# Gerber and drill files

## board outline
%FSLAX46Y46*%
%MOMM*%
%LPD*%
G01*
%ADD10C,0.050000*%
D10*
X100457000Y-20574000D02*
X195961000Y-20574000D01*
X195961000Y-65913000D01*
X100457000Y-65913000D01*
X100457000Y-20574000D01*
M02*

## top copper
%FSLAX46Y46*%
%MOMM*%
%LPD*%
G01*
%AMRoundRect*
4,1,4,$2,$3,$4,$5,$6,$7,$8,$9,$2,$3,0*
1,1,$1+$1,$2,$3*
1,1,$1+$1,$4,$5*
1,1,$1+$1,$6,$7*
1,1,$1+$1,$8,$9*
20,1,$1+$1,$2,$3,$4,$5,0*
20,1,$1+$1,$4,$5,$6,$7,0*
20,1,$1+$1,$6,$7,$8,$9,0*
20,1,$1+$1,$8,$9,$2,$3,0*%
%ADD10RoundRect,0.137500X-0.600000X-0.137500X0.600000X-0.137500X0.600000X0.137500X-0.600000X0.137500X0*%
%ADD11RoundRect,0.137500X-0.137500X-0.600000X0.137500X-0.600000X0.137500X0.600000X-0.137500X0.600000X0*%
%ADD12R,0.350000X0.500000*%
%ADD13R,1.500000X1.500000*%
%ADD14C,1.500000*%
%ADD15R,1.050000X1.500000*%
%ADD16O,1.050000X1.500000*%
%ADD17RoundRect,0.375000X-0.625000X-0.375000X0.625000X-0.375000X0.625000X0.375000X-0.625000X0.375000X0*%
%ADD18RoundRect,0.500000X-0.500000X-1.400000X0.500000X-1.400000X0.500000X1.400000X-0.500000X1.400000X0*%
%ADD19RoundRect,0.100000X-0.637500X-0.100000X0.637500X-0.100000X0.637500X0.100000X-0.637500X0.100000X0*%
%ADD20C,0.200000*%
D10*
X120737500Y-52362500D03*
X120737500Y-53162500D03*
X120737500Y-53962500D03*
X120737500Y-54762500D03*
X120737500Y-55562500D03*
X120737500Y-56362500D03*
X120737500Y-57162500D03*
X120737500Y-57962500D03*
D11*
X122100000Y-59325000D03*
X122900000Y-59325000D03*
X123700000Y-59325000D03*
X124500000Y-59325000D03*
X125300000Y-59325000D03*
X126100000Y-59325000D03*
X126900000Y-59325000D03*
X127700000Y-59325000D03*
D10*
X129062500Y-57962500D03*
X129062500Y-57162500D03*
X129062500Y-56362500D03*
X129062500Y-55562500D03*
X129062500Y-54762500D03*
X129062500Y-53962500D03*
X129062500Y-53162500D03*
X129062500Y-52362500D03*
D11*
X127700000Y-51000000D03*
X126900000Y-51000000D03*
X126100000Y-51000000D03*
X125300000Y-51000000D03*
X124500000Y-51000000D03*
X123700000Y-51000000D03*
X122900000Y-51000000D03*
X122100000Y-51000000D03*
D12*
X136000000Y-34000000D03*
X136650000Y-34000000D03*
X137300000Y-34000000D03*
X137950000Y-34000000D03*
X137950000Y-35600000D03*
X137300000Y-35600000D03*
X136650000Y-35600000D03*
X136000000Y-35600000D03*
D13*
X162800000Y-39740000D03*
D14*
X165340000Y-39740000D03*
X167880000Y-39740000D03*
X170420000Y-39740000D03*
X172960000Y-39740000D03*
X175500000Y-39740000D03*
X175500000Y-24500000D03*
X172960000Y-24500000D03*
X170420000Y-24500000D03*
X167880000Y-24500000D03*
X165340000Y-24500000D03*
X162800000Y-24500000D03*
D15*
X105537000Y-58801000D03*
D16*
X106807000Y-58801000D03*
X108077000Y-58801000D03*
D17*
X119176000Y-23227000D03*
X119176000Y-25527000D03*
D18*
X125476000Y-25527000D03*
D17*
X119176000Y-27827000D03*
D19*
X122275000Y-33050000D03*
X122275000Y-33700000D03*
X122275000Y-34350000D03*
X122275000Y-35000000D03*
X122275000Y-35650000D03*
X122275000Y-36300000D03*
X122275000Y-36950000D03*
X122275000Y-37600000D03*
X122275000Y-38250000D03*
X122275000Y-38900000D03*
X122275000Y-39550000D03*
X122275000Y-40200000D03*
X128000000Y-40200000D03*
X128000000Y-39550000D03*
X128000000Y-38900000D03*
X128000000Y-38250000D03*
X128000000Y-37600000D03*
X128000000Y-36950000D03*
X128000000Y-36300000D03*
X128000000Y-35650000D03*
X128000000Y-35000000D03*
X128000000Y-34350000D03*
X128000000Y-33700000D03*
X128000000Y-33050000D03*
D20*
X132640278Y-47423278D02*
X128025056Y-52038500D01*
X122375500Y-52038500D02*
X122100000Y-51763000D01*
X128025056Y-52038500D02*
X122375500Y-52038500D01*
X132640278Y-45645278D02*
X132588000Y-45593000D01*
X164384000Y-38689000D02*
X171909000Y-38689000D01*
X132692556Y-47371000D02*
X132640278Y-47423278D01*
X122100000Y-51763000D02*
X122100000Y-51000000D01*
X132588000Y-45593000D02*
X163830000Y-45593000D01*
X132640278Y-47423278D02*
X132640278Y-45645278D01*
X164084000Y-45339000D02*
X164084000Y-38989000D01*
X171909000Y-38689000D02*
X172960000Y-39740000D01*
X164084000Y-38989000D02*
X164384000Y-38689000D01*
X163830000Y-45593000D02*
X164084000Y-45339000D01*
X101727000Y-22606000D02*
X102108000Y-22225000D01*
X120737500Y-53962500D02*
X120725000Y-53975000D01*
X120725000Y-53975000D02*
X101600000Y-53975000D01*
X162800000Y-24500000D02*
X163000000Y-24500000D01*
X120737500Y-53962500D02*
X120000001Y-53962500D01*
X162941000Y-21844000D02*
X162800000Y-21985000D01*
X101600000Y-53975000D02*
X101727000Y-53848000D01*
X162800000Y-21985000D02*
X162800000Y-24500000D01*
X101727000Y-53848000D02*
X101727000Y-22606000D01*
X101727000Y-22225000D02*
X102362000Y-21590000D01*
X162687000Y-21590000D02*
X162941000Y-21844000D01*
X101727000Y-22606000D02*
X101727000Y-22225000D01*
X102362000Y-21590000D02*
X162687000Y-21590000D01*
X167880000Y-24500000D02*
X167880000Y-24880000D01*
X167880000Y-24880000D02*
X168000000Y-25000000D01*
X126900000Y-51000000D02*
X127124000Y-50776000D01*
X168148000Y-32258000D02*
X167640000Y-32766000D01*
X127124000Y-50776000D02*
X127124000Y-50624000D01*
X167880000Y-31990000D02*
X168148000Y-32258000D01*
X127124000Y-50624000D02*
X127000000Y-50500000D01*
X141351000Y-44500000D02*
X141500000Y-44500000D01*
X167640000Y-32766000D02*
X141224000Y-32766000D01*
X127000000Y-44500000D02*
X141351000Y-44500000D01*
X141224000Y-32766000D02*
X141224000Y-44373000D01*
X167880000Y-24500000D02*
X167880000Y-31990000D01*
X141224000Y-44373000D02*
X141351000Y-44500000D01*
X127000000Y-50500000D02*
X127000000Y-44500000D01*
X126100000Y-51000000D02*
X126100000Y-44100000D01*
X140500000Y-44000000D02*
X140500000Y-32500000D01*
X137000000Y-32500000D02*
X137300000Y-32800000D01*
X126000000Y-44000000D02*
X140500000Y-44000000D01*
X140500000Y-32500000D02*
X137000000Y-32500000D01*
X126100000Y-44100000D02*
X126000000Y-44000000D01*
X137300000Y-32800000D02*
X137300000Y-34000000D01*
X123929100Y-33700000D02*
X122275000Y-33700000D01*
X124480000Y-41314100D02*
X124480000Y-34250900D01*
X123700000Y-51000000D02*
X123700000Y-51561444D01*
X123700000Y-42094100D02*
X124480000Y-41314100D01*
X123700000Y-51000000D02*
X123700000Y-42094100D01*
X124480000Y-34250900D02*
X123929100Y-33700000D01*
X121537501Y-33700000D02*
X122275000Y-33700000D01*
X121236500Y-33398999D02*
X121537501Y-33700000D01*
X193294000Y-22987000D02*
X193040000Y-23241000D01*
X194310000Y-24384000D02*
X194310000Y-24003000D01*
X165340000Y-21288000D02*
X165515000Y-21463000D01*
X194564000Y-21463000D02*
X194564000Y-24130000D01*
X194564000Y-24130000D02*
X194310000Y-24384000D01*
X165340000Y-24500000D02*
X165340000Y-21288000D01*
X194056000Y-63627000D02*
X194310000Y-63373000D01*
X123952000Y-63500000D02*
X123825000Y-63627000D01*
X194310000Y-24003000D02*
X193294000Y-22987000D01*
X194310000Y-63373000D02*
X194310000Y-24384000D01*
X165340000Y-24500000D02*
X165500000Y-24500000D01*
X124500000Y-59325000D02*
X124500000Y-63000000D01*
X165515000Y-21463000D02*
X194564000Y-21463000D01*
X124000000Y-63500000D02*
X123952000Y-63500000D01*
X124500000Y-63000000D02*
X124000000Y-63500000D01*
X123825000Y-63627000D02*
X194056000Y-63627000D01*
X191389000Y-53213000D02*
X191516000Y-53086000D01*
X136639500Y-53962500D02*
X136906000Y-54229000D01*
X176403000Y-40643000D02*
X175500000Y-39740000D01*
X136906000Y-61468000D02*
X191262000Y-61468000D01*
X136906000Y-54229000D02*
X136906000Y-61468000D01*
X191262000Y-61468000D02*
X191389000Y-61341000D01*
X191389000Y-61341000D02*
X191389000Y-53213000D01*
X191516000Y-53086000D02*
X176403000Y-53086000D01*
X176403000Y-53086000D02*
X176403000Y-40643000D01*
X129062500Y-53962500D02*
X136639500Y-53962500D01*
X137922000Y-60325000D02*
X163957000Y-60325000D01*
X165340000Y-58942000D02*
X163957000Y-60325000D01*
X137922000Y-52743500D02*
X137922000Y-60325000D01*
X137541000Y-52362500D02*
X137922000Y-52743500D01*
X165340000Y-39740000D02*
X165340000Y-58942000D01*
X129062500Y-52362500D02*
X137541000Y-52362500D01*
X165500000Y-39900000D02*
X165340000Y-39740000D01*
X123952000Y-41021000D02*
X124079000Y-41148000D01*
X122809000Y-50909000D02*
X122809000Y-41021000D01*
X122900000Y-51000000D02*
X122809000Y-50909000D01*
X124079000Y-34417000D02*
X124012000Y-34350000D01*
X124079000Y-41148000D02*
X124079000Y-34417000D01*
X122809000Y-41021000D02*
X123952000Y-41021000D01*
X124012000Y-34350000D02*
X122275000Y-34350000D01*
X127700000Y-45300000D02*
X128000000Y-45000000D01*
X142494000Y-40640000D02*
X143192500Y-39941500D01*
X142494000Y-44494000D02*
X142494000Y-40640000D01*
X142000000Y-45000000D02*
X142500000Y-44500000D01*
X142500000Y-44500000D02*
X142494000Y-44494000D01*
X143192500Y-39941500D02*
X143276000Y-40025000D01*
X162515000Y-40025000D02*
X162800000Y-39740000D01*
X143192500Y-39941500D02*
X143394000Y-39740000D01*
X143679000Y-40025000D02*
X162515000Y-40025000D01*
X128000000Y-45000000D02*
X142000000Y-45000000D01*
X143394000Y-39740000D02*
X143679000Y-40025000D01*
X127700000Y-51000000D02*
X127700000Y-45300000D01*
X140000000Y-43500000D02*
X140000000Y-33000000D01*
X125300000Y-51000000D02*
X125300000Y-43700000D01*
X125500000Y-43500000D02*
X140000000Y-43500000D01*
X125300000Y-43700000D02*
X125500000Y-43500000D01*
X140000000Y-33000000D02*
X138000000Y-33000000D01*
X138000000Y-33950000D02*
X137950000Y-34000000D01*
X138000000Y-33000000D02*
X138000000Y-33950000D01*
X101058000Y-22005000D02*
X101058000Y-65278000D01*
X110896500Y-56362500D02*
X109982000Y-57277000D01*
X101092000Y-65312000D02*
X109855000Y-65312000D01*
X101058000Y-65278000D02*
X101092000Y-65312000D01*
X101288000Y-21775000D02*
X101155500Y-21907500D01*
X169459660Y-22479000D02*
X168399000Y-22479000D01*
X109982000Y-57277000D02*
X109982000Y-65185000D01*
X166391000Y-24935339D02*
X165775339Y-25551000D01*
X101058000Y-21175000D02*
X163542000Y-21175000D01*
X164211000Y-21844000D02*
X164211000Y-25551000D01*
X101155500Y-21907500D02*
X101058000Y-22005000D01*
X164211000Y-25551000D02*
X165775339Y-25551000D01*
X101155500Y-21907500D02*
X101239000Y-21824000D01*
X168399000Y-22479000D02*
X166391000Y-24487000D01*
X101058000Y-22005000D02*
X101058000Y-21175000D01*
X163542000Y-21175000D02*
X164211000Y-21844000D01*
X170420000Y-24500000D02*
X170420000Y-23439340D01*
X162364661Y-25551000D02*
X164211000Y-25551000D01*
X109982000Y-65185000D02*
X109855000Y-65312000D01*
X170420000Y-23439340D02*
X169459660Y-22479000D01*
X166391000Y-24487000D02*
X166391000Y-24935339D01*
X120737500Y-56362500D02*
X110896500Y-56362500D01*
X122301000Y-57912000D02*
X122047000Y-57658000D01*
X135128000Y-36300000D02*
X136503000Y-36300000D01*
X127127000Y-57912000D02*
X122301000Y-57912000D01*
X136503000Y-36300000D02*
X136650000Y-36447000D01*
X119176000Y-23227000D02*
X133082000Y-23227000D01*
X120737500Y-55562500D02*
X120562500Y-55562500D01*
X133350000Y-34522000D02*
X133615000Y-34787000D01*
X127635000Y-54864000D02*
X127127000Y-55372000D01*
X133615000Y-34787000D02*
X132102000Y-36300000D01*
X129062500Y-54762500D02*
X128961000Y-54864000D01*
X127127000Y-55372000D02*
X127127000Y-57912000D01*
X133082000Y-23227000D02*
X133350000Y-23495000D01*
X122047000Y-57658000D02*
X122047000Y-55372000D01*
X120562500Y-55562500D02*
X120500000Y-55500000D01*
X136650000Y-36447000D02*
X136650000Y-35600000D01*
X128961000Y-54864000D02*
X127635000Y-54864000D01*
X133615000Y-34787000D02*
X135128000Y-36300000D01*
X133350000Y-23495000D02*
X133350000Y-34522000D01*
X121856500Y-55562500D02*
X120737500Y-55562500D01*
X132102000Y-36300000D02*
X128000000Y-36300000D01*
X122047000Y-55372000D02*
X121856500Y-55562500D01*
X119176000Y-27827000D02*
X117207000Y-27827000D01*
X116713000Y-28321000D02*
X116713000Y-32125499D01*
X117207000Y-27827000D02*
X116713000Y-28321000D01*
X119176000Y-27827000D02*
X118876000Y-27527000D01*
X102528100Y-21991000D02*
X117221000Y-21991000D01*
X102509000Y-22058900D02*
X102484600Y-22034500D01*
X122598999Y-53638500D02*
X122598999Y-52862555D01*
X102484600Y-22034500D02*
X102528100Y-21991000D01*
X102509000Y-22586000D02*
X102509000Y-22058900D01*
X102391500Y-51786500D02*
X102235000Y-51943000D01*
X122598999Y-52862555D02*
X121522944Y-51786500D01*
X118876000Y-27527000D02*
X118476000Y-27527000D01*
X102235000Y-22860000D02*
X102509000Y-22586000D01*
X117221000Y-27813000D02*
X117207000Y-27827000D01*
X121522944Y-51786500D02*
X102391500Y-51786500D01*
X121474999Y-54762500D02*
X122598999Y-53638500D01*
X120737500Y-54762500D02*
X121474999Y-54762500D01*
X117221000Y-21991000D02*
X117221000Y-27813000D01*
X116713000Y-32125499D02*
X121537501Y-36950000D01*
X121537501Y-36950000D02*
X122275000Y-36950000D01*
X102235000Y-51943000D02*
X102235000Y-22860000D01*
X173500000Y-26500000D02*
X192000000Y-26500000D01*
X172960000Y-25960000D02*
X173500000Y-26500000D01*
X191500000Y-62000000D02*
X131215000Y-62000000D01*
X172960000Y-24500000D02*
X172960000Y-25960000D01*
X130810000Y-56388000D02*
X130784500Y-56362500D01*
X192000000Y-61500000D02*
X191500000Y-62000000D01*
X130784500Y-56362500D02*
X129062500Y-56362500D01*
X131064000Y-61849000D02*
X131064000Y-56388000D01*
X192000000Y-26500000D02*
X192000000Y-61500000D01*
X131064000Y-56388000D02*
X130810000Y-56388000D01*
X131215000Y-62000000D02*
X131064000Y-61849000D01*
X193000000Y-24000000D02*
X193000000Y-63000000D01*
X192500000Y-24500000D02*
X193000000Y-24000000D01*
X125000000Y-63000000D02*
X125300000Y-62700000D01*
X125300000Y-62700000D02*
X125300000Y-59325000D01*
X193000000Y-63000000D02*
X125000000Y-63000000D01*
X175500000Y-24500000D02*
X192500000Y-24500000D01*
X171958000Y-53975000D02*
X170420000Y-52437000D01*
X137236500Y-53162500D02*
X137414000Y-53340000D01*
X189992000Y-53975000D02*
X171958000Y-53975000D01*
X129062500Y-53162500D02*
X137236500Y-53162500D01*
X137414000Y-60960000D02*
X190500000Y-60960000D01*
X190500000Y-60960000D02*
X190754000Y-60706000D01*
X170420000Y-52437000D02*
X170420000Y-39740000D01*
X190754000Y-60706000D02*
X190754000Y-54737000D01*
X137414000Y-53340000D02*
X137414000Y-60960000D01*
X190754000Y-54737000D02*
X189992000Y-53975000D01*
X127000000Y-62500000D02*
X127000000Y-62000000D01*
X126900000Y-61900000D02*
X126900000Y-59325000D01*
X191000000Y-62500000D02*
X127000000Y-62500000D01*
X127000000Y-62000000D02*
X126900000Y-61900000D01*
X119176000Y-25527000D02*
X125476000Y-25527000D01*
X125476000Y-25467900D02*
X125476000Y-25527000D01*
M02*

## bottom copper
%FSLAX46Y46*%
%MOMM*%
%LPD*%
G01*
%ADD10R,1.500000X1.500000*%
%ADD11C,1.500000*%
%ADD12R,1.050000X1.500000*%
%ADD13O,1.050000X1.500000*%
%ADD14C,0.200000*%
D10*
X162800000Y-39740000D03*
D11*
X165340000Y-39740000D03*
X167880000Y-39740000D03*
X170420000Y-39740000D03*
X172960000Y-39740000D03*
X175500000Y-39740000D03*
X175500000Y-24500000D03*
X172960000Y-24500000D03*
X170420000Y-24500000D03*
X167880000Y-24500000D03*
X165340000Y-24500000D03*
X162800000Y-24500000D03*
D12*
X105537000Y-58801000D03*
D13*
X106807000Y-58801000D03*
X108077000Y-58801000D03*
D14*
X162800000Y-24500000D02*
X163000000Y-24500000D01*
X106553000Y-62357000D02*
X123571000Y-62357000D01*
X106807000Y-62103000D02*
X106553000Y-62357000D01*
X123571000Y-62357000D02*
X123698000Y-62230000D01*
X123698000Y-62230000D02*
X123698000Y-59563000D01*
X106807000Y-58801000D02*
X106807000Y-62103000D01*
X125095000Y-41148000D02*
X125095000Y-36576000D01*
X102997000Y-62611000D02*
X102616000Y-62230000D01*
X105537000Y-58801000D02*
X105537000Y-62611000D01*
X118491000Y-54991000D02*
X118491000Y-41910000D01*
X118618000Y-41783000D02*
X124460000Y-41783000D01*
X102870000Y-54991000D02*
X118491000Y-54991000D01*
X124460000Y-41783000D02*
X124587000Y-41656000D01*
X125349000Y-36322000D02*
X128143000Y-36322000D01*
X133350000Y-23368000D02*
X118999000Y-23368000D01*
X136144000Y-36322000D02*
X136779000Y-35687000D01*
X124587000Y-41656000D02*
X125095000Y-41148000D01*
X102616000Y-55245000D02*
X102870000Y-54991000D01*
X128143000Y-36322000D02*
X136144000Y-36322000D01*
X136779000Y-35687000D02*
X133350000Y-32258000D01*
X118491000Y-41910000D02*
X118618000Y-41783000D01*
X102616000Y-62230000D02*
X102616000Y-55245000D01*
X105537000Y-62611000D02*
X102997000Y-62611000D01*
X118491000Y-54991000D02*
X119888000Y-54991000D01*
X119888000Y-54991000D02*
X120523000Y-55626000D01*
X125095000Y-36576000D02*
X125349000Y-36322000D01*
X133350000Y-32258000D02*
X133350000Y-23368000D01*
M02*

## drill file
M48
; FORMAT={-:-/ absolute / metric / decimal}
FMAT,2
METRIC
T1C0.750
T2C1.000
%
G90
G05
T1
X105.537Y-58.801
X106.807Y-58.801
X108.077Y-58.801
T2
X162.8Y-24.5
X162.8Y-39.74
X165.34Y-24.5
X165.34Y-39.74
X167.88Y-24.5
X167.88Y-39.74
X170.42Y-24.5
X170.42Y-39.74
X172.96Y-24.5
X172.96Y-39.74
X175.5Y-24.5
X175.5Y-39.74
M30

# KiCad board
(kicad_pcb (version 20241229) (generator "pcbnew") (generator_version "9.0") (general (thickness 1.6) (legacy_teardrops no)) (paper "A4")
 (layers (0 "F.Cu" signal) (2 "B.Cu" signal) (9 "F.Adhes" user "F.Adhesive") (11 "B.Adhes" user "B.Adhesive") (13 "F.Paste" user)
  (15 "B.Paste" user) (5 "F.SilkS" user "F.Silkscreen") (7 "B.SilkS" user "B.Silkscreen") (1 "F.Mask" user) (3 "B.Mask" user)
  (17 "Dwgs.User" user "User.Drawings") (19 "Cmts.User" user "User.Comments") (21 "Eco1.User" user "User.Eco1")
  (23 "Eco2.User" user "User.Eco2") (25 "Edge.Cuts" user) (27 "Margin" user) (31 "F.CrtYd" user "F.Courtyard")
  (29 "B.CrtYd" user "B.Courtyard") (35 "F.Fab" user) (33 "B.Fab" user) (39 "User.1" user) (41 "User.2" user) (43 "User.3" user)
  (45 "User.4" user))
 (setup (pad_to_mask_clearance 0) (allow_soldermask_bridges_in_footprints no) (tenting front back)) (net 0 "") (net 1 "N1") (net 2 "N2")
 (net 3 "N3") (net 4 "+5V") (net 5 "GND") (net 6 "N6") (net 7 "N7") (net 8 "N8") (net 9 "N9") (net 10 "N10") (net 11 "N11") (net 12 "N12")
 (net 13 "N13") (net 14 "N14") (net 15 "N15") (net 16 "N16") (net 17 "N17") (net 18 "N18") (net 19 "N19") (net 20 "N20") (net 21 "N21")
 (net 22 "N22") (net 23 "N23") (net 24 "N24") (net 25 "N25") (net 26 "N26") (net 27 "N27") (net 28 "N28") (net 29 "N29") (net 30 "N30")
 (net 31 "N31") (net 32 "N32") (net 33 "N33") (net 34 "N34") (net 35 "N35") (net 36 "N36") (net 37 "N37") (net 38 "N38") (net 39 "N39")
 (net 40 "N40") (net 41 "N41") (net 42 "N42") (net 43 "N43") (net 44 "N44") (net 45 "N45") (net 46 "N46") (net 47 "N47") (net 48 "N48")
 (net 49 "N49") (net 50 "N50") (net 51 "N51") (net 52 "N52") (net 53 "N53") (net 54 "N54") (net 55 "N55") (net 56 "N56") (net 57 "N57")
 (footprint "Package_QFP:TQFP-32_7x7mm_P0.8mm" (layer "F.Cu") (at 124.9 55.1625)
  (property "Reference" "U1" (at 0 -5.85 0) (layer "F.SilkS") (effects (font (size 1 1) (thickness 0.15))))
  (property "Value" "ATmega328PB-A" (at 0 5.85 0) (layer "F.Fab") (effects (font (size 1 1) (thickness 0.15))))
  (pad "1" smd roundrect (at -4.1625 -2.8) (size 1.475 0.55) (layers "F.Cu" "F.Mask" "F.Paste") (roundrect_rratio 0.25) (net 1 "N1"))
  (pad "2" smd roundrect (at -4.1625 -2) (size 1.475 0.55) (layers "F.Cu" "F.Mask" "F.Paste") (roundrect_rratio 0.25) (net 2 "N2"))
  (pad "3" smd roundrect (at -4.1625 -1.2) (size 1.475 0.55) (layers "F.Cu" "F.Mask" "F.Paste") (roundrect_rratio 0.25) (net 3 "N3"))
  (pad "4" smd roundrect (at -4.1625 -0.4) (size 1.475 0.55) (layers "F.Cu" "F.Mask" "F.Paste") (roundrect_rratio 0.25) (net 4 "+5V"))
  (pad "5" smd roundrect (at -4.1625 0.4) (size 1.475 0.55) (layers "F.Cu" "F.Mask" "F.Paste") (roundrect_rratio 0.25) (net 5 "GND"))
  (pad "6" smd roundrect (at -4.1625 1.2) (size 1.475 0.55) (layers "F.Cu" "F.Mask" "F.Paste") (roundrect_rratio 0.25) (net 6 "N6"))
  (pad "7" smd roundrect (at -4.1625 2) (size 1.475 0.55) (layers "F.Cu" "F.Mask" "F.Paste") (roundrect_rratio 0.25) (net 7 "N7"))
  (pad "8" smd roundrect (at -4.1625 2.8) (size 1.475 0.55) (layers "F.Cu" "F.Mask" "F.Paste") (roundrect_rratio 0.25) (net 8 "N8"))
  (pad "9" smd roundrect (at -2.8 4.1625) (size 0.55 1.475) (layers "F.Cu" "F.Mask" "F.Paste") (roundrect_rratio 0.25) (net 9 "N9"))
  (pad "10" smd roundrect (at -2 4.1625) (size 0.55 1.475) (layers "F.Cu" "F.Mask" "F.Paste") (roundrect_rratio 0.25) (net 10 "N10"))
  (pad "11" smd roundrect (at -1.2 4.1625) (size 0.55 1.475) (layers "F.Cu" "F.Mask" "F.Paste") (roundrect_rratio 0.25) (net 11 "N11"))
  (pad "12" smd roundrect (at -0.4 4.1625) (size 0.55 1.475) (layers "F.Cu" "F.Mask" "F.Paste") (roundrect_rratio 0.25) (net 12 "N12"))
  (pad "13" smd roundrect (at 0.4 4.1625) (size 0.55 1.475) (layers "F.Cu" "F.Mask" "F.Paste") (roundrect_rratio 0.25) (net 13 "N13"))
  (pad "14" smd roundrect (at 1.2 4.1625) (size 0.55 1.475) (layers "F.Cu" "F.Mask" "F.Paste") (roundrect_rratio 0.25) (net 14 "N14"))
  (pad "15" smd roundrect (at 2 4.1625) (size 0.55 1.475) (layers "F.Cu" "F.Mask" "F.Paste") (roundrect_rratio 0.25) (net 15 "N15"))
  (pad "16" smd roundrect (at 2.8 4.1625) (size 0.55 1.475) (layers "F.Cu" "F.Mask" "F.Paste") (roundrect_rratio 0.25) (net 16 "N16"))
  (pad "17" smd roundrect (at 4.1625 2.8) (size 1.475 0.55) (layers "F.Cu" "F.Mask" "F.Paste") (roundrect_rratio 0.25) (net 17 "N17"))
  (pad "18" smd roundrect (at 4.1625 2) (size 1.475 0.55) (layers "F.Cu" "F.Mask" "F.Paste") (roundrect_rratio 0.25) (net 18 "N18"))
  (pad "19" smd roundrect (at 4.1625 1.2) (size 1.475 0.55) (layers "F.Cu" "F.Mask" "F.Paste") (roundrect_rratio 0.25) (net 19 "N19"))
  (pad "20" smd roundrect (at 4.1625 0.4) (size 1.475 0.55) (layers "F.Cu" "F.Mask" "F.Paste") (roundrect_rratio 0.25) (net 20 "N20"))
  (pad "21" smd roundrect (at 4.1625 -0.4) (size 1.475 0.55) (layers "F.Cu" "F.Mask" "F.Paste") (roundrect_rratio 0.25) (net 5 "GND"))
  (pad "22" smd roundrect (at 4.1625 -1.2) (size 1.475 0.55) (layers "F.Cu" "F.Mask" "F.Paste") (roundrect_rratio 0.25) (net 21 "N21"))
  (pad "23" smd roundrect (at 4.1625 -2) (size 1.475 0.55) (layers "F.Cu" "F.Mask" "F.Paste") (roundrect_rratio 0.25) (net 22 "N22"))
  (pad "24" smd roundrect (at 4.1625 -2.8) (size 1.475 0.55) (layers "F.Cu" "F.Mask" "F.Paste") (roundrect_rratio 0.25) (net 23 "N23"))
  (pad "25" smd roundrect (at 2.8 -4.1625) (size 0.55 1.475) (layers "F.Cu" "F.Mask" "F.Paste") (roundrect_rratio 0.25) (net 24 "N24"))
  (pad "26" smd roundrect (at 2 -4.1625) (size 0.55 1.475) (layers "F.Cu" "F.Mask" "F.Paste") (roundrect_rratio 0.25) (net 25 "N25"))
  (pad "27" smd roundrect (at 1.2 -4.1625) (size 0.55 1.475) (layers "F.Cu" "F.Mask" "F.Paste") (roundrect_rratio 0.25) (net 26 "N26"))
  (pad "28" smd roundrect (at 0.4 -4.1625) (size 0.55 1.475) (layers "F.Cu" "F.Mask" "F.Paste") (roundrect_rratio 0.25) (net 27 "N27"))
  (pad "29" smd roundrect (at -0.4 -4.1625) (size 0.55 1.475) (layers "F.Cu" "F.Mask" "F.Paste") (roundrect_rratio 0.25) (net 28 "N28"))
  (pad "30" smd roundrect (at -1.2 -4.1625) (size 0.55 1.475) (layers "F.Cu" "F.Mask" "F.Paste") (roundrect_rratio 0.25) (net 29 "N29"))
  (pad "31" smd roundrect (at -2 -4.1625) (size 0.55 1.475) (layers "F.Cu" "F.Mask" "F.Paste") (roundrect_rratio 0.25) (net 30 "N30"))
  (pad "32" smd roundrect (at -2.8 -4.1625) (size 0.55 1.475) (layers "F.Cu" "F.Mask" "F.Paste") (roundrect_rratio 0.25) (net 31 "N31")))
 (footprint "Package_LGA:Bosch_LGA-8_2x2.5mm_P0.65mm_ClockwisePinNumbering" (layer "F.Cu") (at 136.975 34.8)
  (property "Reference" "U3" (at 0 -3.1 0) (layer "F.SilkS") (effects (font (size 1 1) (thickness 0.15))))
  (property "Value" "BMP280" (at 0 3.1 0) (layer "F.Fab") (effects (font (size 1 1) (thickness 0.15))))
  (pad "1" smd rect (at -0.975 -0.8 90) (size 0.5 0.35) (layers "F.Cu" "F.Mask" "F.Paste") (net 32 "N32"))
  (pad "2" smd rect (at -0.325 -0.8 90) (size 0.5 0.35) (layers "F.Cu" "F.Mask" "F.Paste") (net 32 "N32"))
  (pad "3" smd rect (at 0.325 -0.8 90) (size 0.5 0.35) (layers "F.Cu" "F.Mask" "F.Paste") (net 26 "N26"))
  (pad "4" smd rect (at 0.975 -0.8 90) (size 0.5 0.35) (layers "F.Cu" "F.Mask" "F.Paste") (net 27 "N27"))
  (pad "5" smd rect (at 0.975 0.8 90) (size 0.5 0.35) (layers "F.Cu" "F.Mask" "F.Paste") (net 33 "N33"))
  (pad "6" smd rect (at 0.325 0.8 90) (size 0.5 0.35) (layers "F.Cu" "F.Mask" "F.Paste") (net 33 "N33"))
  (pad "7" smd rect (at -0.325 0.8 90) (size 0.5 0.35) (layers "F.Cu" "F.Mask" "F.Paste") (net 5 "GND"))
  (pad "8" smd rect (at -0.975 0.8 90) (size 0.5 0.35) (layers "F.Cu" "F.Mask" "F.Paste") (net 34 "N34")))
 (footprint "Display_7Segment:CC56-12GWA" (layer "F.Cu") (at 162.8 39.74 90)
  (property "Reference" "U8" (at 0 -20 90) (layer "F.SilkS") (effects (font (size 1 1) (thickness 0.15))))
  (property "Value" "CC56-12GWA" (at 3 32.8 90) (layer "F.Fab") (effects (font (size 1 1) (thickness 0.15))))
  (pad "1" thru_hole rect (at 0 0 90) (size 1.5 1.5) (drill 1) (layers "*.Cu" "*.Mask") (remove_unused_layers no) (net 24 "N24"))
  (pad "2" thru_hole circle (at 0 2.54 90) (size 1.5 1.5) (drill 1) (layers "*.Cu" "*.Mask") (remove_unused_layers no) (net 23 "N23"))
  (pad "3" thru_hole circle (at 0 5.08 90) (size 1.5 1.5) (drill 1) (layers "*.Cu" "*.Mask") (remove_unused_layers no) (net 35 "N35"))
  (pad "4" thru_hole circle (at 0 7.62 90) (size 1.5 1.5) (drill 1) (layers "*.Cu" "*.Mask") (remove_unused_layers no) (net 22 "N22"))
  (pad "5" thru_hole circle (at 0 10.16 90) (size 1.5 1.5) (drill 1) (layers "*.Cu" "*.Mask") (remove_unused_layers no) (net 31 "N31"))
  (pad "6" thru_hole circle (at 0 12.7 90) (size 1.5 1.5) (drill 1) (layers "*.Cu" "*.Mask") (remove_unused_layers no) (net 21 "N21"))
  (pad "7" thru_hole circle (at 15.24 12.7 90) (size 1.5 1.5) (drill 1) (layers "*.Cu" "*.Mask") (remove_unused_layers no) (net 13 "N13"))
  (pad "8" thru_hole circle (at 15.24 10.16 90) (size 1.5 1.5) (drill 1) (layers "*.Cu" "*.Mask") (remove_unused_layers no) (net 19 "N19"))
  (pad "9" thru_hole circle (at 15.24 7.62 90) (size 1.5 1.5) (drill 1) (layers "*.Cu" "*.Mask") (remove_unused_layers no) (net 6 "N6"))
  (pad "10" thru_hole circle (at 15.24 5.08 90) (size 1.5 1.5) (drill 1) (layers "*.Cu" "*.Mask") (remove_unused_layers no) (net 25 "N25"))
  (pad "11" thru_hole circle (at 15.24 2.54 90) (size 1.5 1.5) (drill 1) (layers "*.Cu" "*.Mask") (remove_unused_layers no) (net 12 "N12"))
  (pad "12" thru_hole circle (at 15.24 0 90) (size 1.5 1.5) (drill 1) (layers "*.Cu" "*.Mask") (remove_unused_layers no) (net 3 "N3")))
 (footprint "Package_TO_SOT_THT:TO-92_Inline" (layer "F.Cu") (at 105.537 58.801)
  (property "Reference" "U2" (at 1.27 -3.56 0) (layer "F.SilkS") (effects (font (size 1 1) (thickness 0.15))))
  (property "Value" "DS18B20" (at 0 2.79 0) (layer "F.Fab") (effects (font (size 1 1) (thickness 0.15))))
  (pad "1" thru_hole rect (at 0 0) (size 1.05 1.5) (drill 0.75) (layers "*.Cu" "*.Mask") (remove_unused_layers no) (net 5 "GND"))
  (pad "2" thru_hole oval (at 1.27 0) (size 1.05 1.5) (drill 0.75) (layers "*.Cu" "*.Mask") (remove_unused_layers no) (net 11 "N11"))
  (pad "3" thru_hole oval (at 2.54 0) (size 1.05 1.5) (drill 0.75) (layers "*.Cu" "*.Mask") (remove_unused_layers no) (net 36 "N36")))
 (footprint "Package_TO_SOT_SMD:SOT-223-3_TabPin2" (layer "F.Cu") (at 122.326 25.527)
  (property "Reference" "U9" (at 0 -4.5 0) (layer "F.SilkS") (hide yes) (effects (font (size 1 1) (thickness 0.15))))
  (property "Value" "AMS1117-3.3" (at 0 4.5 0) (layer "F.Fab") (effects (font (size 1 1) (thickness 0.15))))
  (pad "1" smd roundrect (at -3.15 -2.3) (size 2 1.5) (layers "F.Cu" "F.Mask" "F.Paste") (roundrect_rratio 0.25) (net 5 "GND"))
  (pad "2" smd roundrect (at -3.15 0) (size 2 1.5) (layers "F.Cu" "F.Mask" "F.Paste") (roundrect_rratio 0.25) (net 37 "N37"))
  (pad "2" smd roundrect (at 3.15 0) (size 2 3.8) (layers "F.Cu" "F.Mask" "F.Paste") (roundrect_rratio 0.25) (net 37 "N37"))
  (pad "3" smd roundrect (at -3.15 2.3) (size 2 1.5) (layers "F.Cu" "F.Mask" "F.Paste") (roundrect_rratio 0.25) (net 4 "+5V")))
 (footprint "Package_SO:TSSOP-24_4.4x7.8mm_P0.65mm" (layer "F.Cu") (at 125.1375 36.625)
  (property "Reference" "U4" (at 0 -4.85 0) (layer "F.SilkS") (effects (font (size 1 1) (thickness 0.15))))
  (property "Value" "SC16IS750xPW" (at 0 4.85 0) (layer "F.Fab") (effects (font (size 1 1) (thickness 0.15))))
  (pad "1" smd roundrect (at -2.8625 -3.575) (size 1.475 0.4) (layers "F.Cu" "F.Mask" "F.Paste") (roundrect_rratio 0.25) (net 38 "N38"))
  (pad "2" smd roundrect (at -2.8625 -2.925) (size 1.475 0.4) (layers "F.Cu" "F.Mask" "F.Paste") (roundrect_rratio 0.25) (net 29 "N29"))
  (pad "3" smd roundrect (at -2.8625 -2.275) (size 1.475 0.4) (layers "F.Cu" "F.Mask" "F.Paste") (roundrect_rratio 0.25) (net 30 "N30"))
  (pad "4" smd roundrect (at -2.8625 -1.625) (size 1.475 0.4) (layers "F.Cu" "F.Mask" "F.Paste") (roundrect_rratio 0.25) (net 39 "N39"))
  (pad "5" smd roundrect (at -2.8625 -0.975) (size 1.475 0.4) (layers "F.Cu" "F.Mask" "F.Paste") (roundrect_rratio 0.25) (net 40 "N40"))
  (pad "6" smd roundrect (at -2.8625 -0.325) (size 1.475 0.4) (layers "F.Cu" "F.Mask" "F.Paste") (roundrect_rratio 0.25) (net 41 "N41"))
  (pad "7" smd roundrect (at -2.8625 0.325) (size 1.475 0.4) (layers "F.Cu" "F.Mask" "F.Paste") (roundrect_rratio 0.25) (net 4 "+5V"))
  (pad "8" smd roundrect (at -2.8625 0.975) (size 1.475 0.4) (layers "F.Cu" "F.Mask" "F.Paste") (roundrect_rratio 0.25) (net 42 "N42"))
  (pad "9" smd roundrect (at -2.8625 1.625) (size 1.475 0.4) (layers "F.Cu" "F.Mask" "F.Paste") (roundrect_rratio 0.25) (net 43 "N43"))
  (pad "10" smd roundrect (at -2.8625 2.275) (size 1.475 0.4) (layers "F.Cu" "F.Mask" "F.Paste") (roundrect_rratio 0.25) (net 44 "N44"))
  (pad "11" smd roundrect (at -2.8625 2.925) (size 1.475 0.4) (layers "F.Cu" "F.Mask" "F.Paste") (roundrect_rratio 0.25) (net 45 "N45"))
  (pad "12" smd roundrect (at -2.8625 3.575) (size 1.475 0.4) (layers "F.Cu" "F.Mask" "F.Paste") (roundrect_rratio 0.25) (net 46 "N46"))
  (pad "13" smd roundrect (at 2.8625 3.575) (size 1.475 0.4) (layers "F.Cu" "F.Mask" "F.Paste") (roundrect_rratio 0.25) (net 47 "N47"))
  (pad "14" smd roundrect (at 2.8625 2.925) (size 1.475 0.4) (layers "F.Cu" "F.Mask" "F.Paste") (roundrect_rratio 0.25) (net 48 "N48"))
  (pad "15" smd roundrect (at 2.8625 2.275) (size 1.475 0.4) (layers "F.Cu" "F.Mask" "F.Paste") (roundrect_rratio 0.25) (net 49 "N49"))
  (pad "16" smd roundrect (at 2.8625 1.625) (size 1.475 0.4) (layers "F.Cu" "F.Mask" "F.Paste") (roundrect_rratio 0.25) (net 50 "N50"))
  (pad "17" smd roundrect (at 2.8625 0.975) (size 1.475 0.4) (layers "F.Cu" "F.Mask" "F.Paste") (roundrect_rratio 0.25) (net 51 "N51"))
  (pad "18" smd roundrect (at 2.8625 0.325) (size 1.475 0.4) (layers "F.Cu" "F.Mask" "F.Paste") (roundrect_rratio 0.25) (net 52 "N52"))
  (pad "19" smd roundrect (at 2.8625 -0.325) (size 1.475 0.4) (layers "F.Cu" "F.Mask" "F.Paste") (roundrect_rratio 0.25) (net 5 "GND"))
  (pad "20" smd roundrect (at 2.8625 -0.975) (size 1.475 0.4) (layers "F.Cu" "F.Mask" "F.Paste") (roundrect_rratio 0.25) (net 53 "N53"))
  (pad "21" smd roundrect (at 2.8625 -1.625) (size 1.475 0.4) (layers "F.Cu" "F.Mask" "F.Paste") (roundrect_rratio 0.25) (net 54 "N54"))
  (pad "22" smd roundrect (at 2.8625 -2.275) (size 1.475 0.4) (layers "F.Cu" "F.Mask" "F.Paste") (roundrect_rratio 0.25) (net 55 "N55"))
  (pad "23" smd roundrect (at 2.8625 -2.925) (size 1.475 0.4) (layers "F.Cu" "F.Mask" "F.Paste") (roundrect_rratio 0.25) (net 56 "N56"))
  (pad "24" smd roundrect (at 2.8625 -3.575) (size 1.475 0.4) (layers "F.Cu" "F.Mask" "F.Paste") (roundrect_rratio 0.25) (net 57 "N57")))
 (gr_rect (start 100.457 20.574) (end 195.961 65.913) (stroke (width 0.05) (type default)) (fill no) (layer "Edge.Cuts"))
 (segment (start 132.640278 47.423278) (end 128.025056 52.0385) (width 0.2) (layer "F.Cu") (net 31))
 (segment (start 122.3755 52.0385) (end 122.1 51.763) (width 0.2) (layer "F.Cu") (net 31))
 (segment (start 128.025056 52.0385) (end 122.3755 52.0385) (width 0.2) (layer "F.Cu") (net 31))
 (segment (start 132.640278 45.645278) (end 132.588 45.593) (width 0.2) (layer "F.Cu") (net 31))
 (segment (start 164.384 38.689) (end 171.909 38.689) (width 0.2) (layer "F.Cu") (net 31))
 (segment (start 132.692556 47.371) (end 132.640278 47.423278) (width 0.2) (layer "F.Cu") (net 31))
 (segment (start 122.1 51.763) (end 122.1 51) (width 0.2) (layer "F.Cu") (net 31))
 (segment (start 132.588 45.593) (end 163.83 45.593) (width 0.2) (layer "F.Cu") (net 31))
 (segment (start 132.640278 47.423278) (end 132.640278 45.645278) (width 0.2) (layer "F.Cu") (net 31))
 (segment (start 164.084 45.339) (end 164.084 38.989) (width 0.2) (layer "F.Cu") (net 31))
 (segment (start 171.909 38.689) (end 172.96 39.74) (width 0.2) (layer "F.Cu") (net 31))
 (segment (start 164.084 38.989) (end 164.384 38.689) (width 0.2) (layer "F.Cu") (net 31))
 (segment (start 163.83 45.593) (end 164.084 45.339) (width 0.2) (layer "F.Cu") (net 31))
 (segment (start 101.727 22.606) (end 102.108 22.225) (width 0.2) (layer "F.Cu") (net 3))
 (segment (start 120.7375 53.9625) (end 120.725 53.975) (width 0.2) (layer "F.Cu") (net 3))
 (segment (start 120.725 53.975) (end 101.6 53.975) (width 0.2) (layer "F.Cu") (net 3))
 (segment (start 162.8 24.5) (end 163 24.5) (width 0.2) (layer "F.Cu") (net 3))
 (segment (start 120.7375 53.9625) (end 120.000001 53.9625) (width 0.2) (layer "F.Cu") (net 3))
 (segment (start 162.941 21.844) (end 162.8 21.985) (width 0.2) (layer "F.Cu") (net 3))
 (segment (start 101.6 53.975) (end 101.727 53.848) (width 0.2) (layer "F.Cu") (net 3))
 (segment (start 162.8 21.985) (end 162.8 24.5) (width 0.2) (layer "F.Cu") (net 3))
 (segment (start 101.727 53.848) (end 101.727 22.606) (width 0.2) (layer "F.Cu") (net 3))
 (segment (start 101.727 22.225) (end 102.362 21.59) (width 0.2) (layer "F.Cu") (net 3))
 (segment (start 162.687 21.59) (end 162.941 21.844) (width 0.2) (layer "F.Cu") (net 3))
 (segment (start 101.727 22.606) (end 101.727 22.225) (width 0.2) (layer "F.Cu") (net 3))
 (segment (start 102.362 21.59) (end 162.687 21.59) (width 0.2) (layer "F.Cu") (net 3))
 (segment (start 162.8 24.5) (end 163 24.5) (width 0.2) (layer "B.Cu") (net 3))
 (segment (start 167.88 24.5) (end 167.88 24.88) (width 0.2) (layer "F.Cu") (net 25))
 (segment (start 167.88 24.88) (end 168 25) (width 0.2) (layer "F.Cu") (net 25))
 (segment (start 126.9 51) (end 127.124 50.776) (width 0.2) (layer "F.Cu") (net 25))
 (segment (start 168.148 32.258) (end 167.64 32.766) (width 0.2) (layer "F.Cu") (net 25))
 (segment (start 127.124 50.776) (end 127.124 50.624) (width 0.2) (layer "F.Cu") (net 25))
 (segment (start 167.88 31.99) (end 168.148 32.258) (width 0.2) (layer "F.Cu") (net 25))
 (segment (start 127.124 50.624) (end 127 50.5) (width 0.2) (layer "F.Cu") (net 25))
 (segment (start 141.351 44.5) (end 141.5 44.5) (width 0.2) (layer "F.Cu") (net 25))
 (segment (start 167.64 32.766) (end 141.224 32.766) (width 0.2) (layer "F.Cu") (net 25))
 (segment (start 127 44.5) (end 141.351 44.5) (width 0.2) (layer "F.Cu") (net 25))
 (segment (start 141.224 32.766) (end 141.224 44.373) (width 0.2) (layer "F.Cu") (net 25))
 (segment (start 167.88 24.5) (end 167.88 31.99) (width 0.2) (layer "F.Cu") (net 25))
 (segment (start 141.224 44.373) (end 141.351 44.5) (width 0.2) (layer "F.Cu") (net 25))
 (segment (start 127 50.5) (end 127 44.5) (width 0.2) (layer "F.Cu") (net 25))
 (segment (start 126.1 51) (end 126.1 44.1) (width 0.2) (layer "F.Cu") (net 26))
 (segment (start 140.5 44) (end 140.5 32.5) (width 0.2) (layer "F.Cu") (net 26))
 (segment (start 137 32.5) (end 137.3 32.8) (width 0.2) (layer "F.Cu") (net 26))
 (segment (start 126 44) (end 140.5 44) (width 0.2) (layer "F.Cu") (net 26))
 (segment (start 140.5 32.5) (end 137 32.5) (width 0.2) (layer "F.Cu") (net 26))
 (segment (start 126.1 44.1) (end 126 44) (width 0.2) (layer "F.Cu") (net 26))
 (segment (start 137.3 32.8) (end 137.3 34) (width 0.2) (layer "F.Cu") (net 26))
 (segment (start 123.9291 33.7) (end 122.275 33.7) (width 0.2) (layer "F.Cu") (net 29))
 (segment (start 124.48 41.3141) (end 124.48 34.2509) (width 0.2) (layer "F.Cu") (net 29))
 (segment (start 123.7 51) (end 123.7 51.561444) (width 0.2) (layer "F.Cu") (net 29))
 (segment (start 123.7 42.0941) (end 124.48 41.3141) (width 0.2) (layer "F.Cu") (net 29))
 (segment (start 123.7 51) (end 123.7 42.0941) (width 0.2) (layer "F.Cu") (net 29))
 (segment (start 124.48 34.2509) (end 123.9291 33.7) (width 0.2) (layer "F.Cu") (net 29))
 (segment (start 121.537501 33.7) (end 122.275 33.7) (width 0.2) (layer "F.Cu") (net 29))
 (segment (start 121.2365 33.398999) (end 121.537501 33.7) (width 0.2) (layer "F.Cu") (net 29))
 (segment (start 193.294 22.987) (end 193.04 23.241) (width 0.2) (layer "F.Cu") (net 12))
 (segment (start 194.31 24.384) (end 194.31 24.003) (width 0.2) (layer "F.Cu") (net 12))
 (segment (start 165.34 21.288) (end 165.515 21.463) (width 0.2) (layer "F.Cu") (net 12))
 (segment (start 194.564 21.463) (end 194.564 24.13) (width 0.2) (layer "F.Cu") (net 12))
 (segment (start 194.564 24.13) (end 194.31 24.384) (width 0.2) (layer "F.Cu") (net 12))
 (segment (start 165.34 24.5) (end 165.34 21.288) (width 0.2) (layer "F.Cu") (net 12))
 (segment (start 194.056 63.627) (end 194.31 63.373) (width 0.2) (layer "F.Cu") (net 12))
 (segment (start 123.952 63.5) (end 123.825 63.627) (width 0.2) (layer "F.Cu") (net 12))
 (segment (start 194.31 24.003) (end 193.294 22.987) (width 0.2) (layer "F.Cu") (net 12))
 (segment (start 194.31 63.373) (end 194.31 24.384) (width 0.2) (layer "F.Cu") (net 12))
 (segment (start 165.34 24.5) (end 165.5 24.5) (width 0.2) (layer "F.Cu") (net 12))
 (segment (start 124.5 59.325) (end 124.5 63) (width 0.2) (layer "F.Cu") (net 12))
 (segment (start 165.515 21.463) (end 194.564 21.463) (width 0.2) (layer "F.Cu") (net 12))
 (segment (start 124 63.5) (end 123.952 63.5) (width 0.2) (layer "F.Cu") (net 12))
 (segment (start 124.5 63) (end 124 63.5) (width 0.2) (layer "F.Cu") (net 12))
 (segment (start 123.825 63.627) (end 194.056 63.627) (width 0.2) (layer "F.Cu") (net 12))
 (segment (start 106.553 62.357) (end 123.571 62.357) (width 0.2) (layer "B.Cu") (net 11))
 (segment (start 106.807 62.103) (end 106.553 62.357) (width 0.2) (layer "B.Cu") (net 11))
 (segment (start 123.571 62.357) (end 123.698 62.23) (width 0.2) (layer "B.Cu") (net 11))
 (segment (start 123.698 62.23) (end 123.698 59.563) (width 0.2) (layer "B.Cu") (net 11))
 (segment (start 106.807 58.801) (end 106.807 62.103) (width 0.2) (layer "B.Cu") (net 11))
 (segment (start 191.389 53.213) (end 191.516 53.086) (width 0.2) (layer "F.Cu") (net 21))
 (segment (start 136.6395 53.9625) (end 136.906 54.229) (width 0.2) (layer "F.Cu") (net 21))
 (segment (start 176.403 40.643) (end 175.5 39.74) (width 0.2) (layer "F.Cu") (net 21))
 (segment (start 136.906 61.468) (end 191.262 61.468) (width 0.2) (layer "F.Cu") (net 21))
 (segment (start 136.906 54.229) (end 136.906 61.468) (width 0.2) (layer "F.Cu") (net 21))
 (segment (start 191.262 61.468) (end 191.389 61.341) (width 0.2) (layer "F.Cu") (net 21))
 (segment (start 191.389 61.341) (end 191.389 53.213) (width 0.2) (layer "F.Cu") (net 21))
 (segment (start 191.516 53.086) (end 176.403 53.086) (width 0.2) (layer "F.Cu") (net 21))
 (segment (start 176.403 53.086) (end 176.403 40.643) (width 0.2) (layer "F.Cu") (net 21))
 (segment (start 129.0625 53.9625) (end 136.6395 53.9625) (width 0.2) (layer "F.Cu") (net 21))
 (segment (start 137.922 60.325) (end 163.957 60.325) (width 0.2) (layer "F.Cu") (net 23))
 (segment (start 165.34 58.942) (end 163.957 60.325) (width 0.2) (layer "F.Cu") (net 23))
 (segment (start 137.922 52.7435) (end 137.922 60.325) (width 0.2) (layer "F.Cu") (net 23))
 (segment (start 137.541 52.3625) (end 137.922 52.7435) (width 0.2) (layer "F.Cu") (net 23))
 (segment (start 165.34 39.74) (end 165.34 58.942) (width 0.2) (layer "F.Cu") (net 23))
 (segment (start 129.0625 52.3625) (end 137.541 52.3625) (width 0.2) (layer "F.Cu") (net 23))
 (segment (start 165.5 39.9) (end 165.34 39.74) (width 0.2) (layer "F.Cu") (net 23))
 (segment (start 123.952 41.021) (end 124.079 41.148) (width 0.2) (layer "F.Cu") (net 30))
 (segment (start 122.809 50.909) (end 122.809 41.021) (width 0.2) (layer "F.Cu") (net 30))
 (segment (start 122.9 51) (end 122.809 50.909) (width 0.2) (layer "F.Cu") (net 30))
 (segment (start 124.079 34.417) (end 124.012 34.35) (width 0.2) (layer "F.Cu") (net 30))
 (segment (start 124.079 41.148) (end 124.079 34.417) (width 0.2) (layer "F.Cu") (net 30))
 (segment (start 122.809 41.021) (end 123.952 41.021) (width 0.2) (layer "F.Cu") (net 30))
 (segment (start 124.012 34.35) (end 122.275 34.35) (width 0.2) (layer "F.Cu") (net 30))
 (segment (start 127.7 45.3) (end 128 45) (width 0.2) (layer "F.Cu") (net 24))
 (segment (start 142.494 40.64) (end 143.1925 39.9415) (width 0.2) (layer "F.Cu") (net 24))
 (segment (start 142.494 44.494) (end 142.494 40.64) (width 0.2) (layer "F.Cu") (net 24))
 (segment (start 142 45) (end 142.5 44.5) (width 0.2) (layer "F.Cu") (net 24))
 (segment (start 142.5 44.5) (end 142.494 44.494) (width 0.2) (layer "F.Cu") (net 24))
 (segment (start 143.1925 39.9415) (end 143.276 40.025) (width 0.2) (layer "F.Cu") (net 24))
 (segment (start 162.515 40.025) (end 162.8 39.74) (width 0.2) (layer "F.Cu") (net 24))
 (segment (start 143.1925 39.9415) (end 143.394 39.74) (width 0.2) (layer "F.Cu") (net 24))
 (segment (start 143.679 40.025) (end 162.515 40.025) (width 0.2) (layer "F.Cu") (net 24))
 (segment (start 128 45) (end 142 45) (width 0.2) (layer "F.Cu") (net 24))
 (segment (start 143.394 39.74) (end 143.679 40.025) (width 0.2) (layer "F.Cu") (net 24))
 (segment (start 127.7 51) (end 127.7 45.3) (width 0.2) (layer "F.Cu") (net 24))
 (segment (start 140 43.5) (end 140 33) (width 0.2) (layer "F.Cu") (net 27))
 (segment (start 125.3 51) (end 125.3 43.7) (width 0.2) (layer "F.Cu") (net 27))
 (segment (start 125.5 43.5) (end 140 43.5) (width 0.2) (layer "F.Cu") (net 27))
 (segment (start 125.3 43.7) (end 125.5 43.5) (width 0.2) (layer "F.Cu") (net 27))
 (segment (start 140 33) (end 138 33) (width 0.2) (layer "F.Cu") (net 27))
 (segment (start 138 33.95) (end 137.95 34) (width 0.2) (layer "F.Cu") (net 27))
 (segment (start 138 33) (end 138 33.95) (width 0.2) (layer "F.Cu") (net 27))
 (segment (start 101.058 22.005) (end 101.058 65.278) (width 0.2) (layer "F.Cu") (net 6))
 (segment (start 110.8965 56.3625) (end 109.982 57.277) (width 0.2) (layer "F.Cu") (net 6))
 (segment (start 101.092 65.312) (end 109.855 65.312) (width 0.2) (layer "F.Cu") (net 6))
 (segment (start 101.058 65.278) (end 101.092 65.312) (width 0.2) (layer "F.Cu") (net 6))
 (segment (start 101.288 21.775) (end 101.1555 21.9075) (width 0.2) (layer "F.Cu") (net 6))
 (segment (start 169.45966 22.479) (end 168.399 22.479) (width 0.2) (layer "F.Cu") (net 6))
 (segment (start 109.982 57.277) (end 109.982 65.185) (width 0.2) (layer "F.Cu") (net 6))
 (segment (start 166.391 24.935339) (end 165.775339 25.551) (width 0.2) (layer "F.Cu") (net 6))
 (segment (start 101.058 21.175) (end 163.542 21.175) (width 0.2) (layer "F.Cu") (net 6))
 (segment (start 164.211 21.844) (end 164.211 25.551) (width 0.2) (layer "F.Cu") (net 6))
 (segment (start 101.1555 21.9075) (end 101.058 22.005) (width 0.2) (layer "F.Cu") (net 6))
 (segment (start 164.211 25.551) (end 165.775339 25.551) (width 0.2) (layer "F.Cu") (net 6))
 (segment (start 101.1555 21.9075) (end 101.239 21.824) (width 0.2) (layer "F.Cu") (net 6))
 (segment (start 168.399 22.479) (end 166.391 24.487) (width 0.2) (layer "F.Cu") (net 6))
 (segment (start 101.058 22.005) (end 101.058 21.175) (width 0.2) (layer "F.Cu") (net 6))
 (segment (start 163.542 21.175) (end 164.211 21.844) (width 0.2) (layer "F.Cu") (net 6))
 (segment (start 170.42 24.5) (end 170.42 23.43934) (width 0.2) (layer "F.Cu") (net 6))
 (segment (start 162.364661 25.551) (end 164.211 25.551) (width 0.2) (layer "F.Cu") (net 6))
 (segment (start 109.982 65.185) (end 109.855 65.312) (width 0.2) (layer "F.Cu") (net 6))
 (segment (start 170.42 23.43934) (end 169.45966 22.479) (width 0.2) (layer "F.Cu") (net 6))
 (segment (start 166.391 24.487) (end 166.391 24.935339) (width 0.2) (layer "F.Cu") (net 6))
 (segment (start 120.7375 56.3625) (end 110.8965 56.3625) (width 0.2) (layer "F.Cu") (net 6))
 (segment (start 122.301 57.912) (end 122.047 57.658) (width 0.2) (layer "F.Cu") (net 5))
 (segment (start 135.128 36.3) (end 136.503 36.3) (width 0.2) (layer "F.Cu") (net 5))
 (segment (start 127.127 57.912) (end 122.301 57.912) (width 0.2) (layer "F.Cu") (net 5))
 (segment (start 136.503 36.3) (end 136.65 36.447) (width 0.2) (layer "F.Cu") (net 5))
 (segment (start 119.176 23.227) (end 133.082 23.227) (width 0.2) (layer "F.Cu") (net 5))
 (segment (start 120.7375 55.5625) (end 120.5625 55.5625) (width 0.2) (layer "F.Cu") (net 5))
 (segment (start 133.35 34.522) (end 133.615 34.787) (width 0.2) (layer "F.Cu") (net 5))
 (segment (start 127.635 54.864) (end 127.127 55.372) (width 0.2) (layer "F.Cu") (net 5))
 (segment (start 133.615 34.787) (end 132.102 36.3) (width 0.2) (layer "F.Cu") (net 5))
 (segment (start 129.0625 54.7625) (end 128.961 54.864) (width 0.2) (layer "F.Cu") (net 5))
 (segment (start 127.127 55.372) (end 127.127 57.912) (width 0.2) (layer "F.Cu") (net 5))
 (segment (start 133.082 23.227) (end 133.35 23.495) (width 0.2) (layer "F.Cu") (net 5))
 (segment (start 122.047 57.658) (end 122.047 55.372) (width 0.2) (layer "F.Cu") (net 5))
 (segment (start 120.5625 55.5625) (end 120.5 55.5) (width 0.2) (layer "F.Cu") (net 5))
 (segment (start 136.65 36.447) (end 136.65 35.6) (width 0.2) (layer "F.Cu") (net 5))
 (segment (start 128.961 54.864) (end 127.635 54.864) (width 0.2) (layer "F.Cu") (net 5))
 (segment (start 133.615 34.787) (end 135.128 36.3) (width 0.2) (layer "F.Cu") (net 5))
 (segment (start 133.35 23.495) (end 133.35 34.522) (width 0.2) (layer "F.Cu") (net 5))
 (segment (start 121.8565 55.5625) (end 120.7375 55.5625) (width 0.2) (layer "F.Cu") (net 5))
 (segment (start 132.102 36.3) (end 128 36.3) (width 0.2) (layer "F.Cu") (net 5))
 (segment (start 122.047 55.372) (end 121.8565 55.5625) (width 0.2) (layer "F.Cu") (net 5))
 (segment (start 125.095 41.148) (end 125.095 36.576) (width 0.2) (layer "B.Cu") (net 5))
 (segment (start 102.997 62.611) (end 102.616 62.23) (width 0.2) (layer "B.Cu") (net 5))
 (segment (start 105.537 58.801) (end 105.537 62.611) (width 0.2) (layer "B.Cu") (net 5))
 (segment (start 118.491 54.991) (end 118.491 41.91) (width 0.2) (layer "B.Cu") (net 5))
 (segment (start 118.618 41.783) (end 124.46 41.783) (width 0.2) (layer "B.Cu") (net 5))
 (segment (start 102.87 54.991) (end 118.491 54.991) (width 0.2) (layer "B.Cu") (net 5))
 (segment (start 124.46 41.783) (end 124.587 41.656) (width 0.2) (layer "B.Cu") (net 5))
 (segment (start 125.349 36.322) (end 128.143 36.322) (width 0.2) (layer "B.Cu") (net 5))
 (segment (start 133.35 23.368) (end 118.999 23.368) (width 0.2) (layer "B.Cu") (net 5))
 (segment (start 136.144 36.322) (end 136.779 35.687) (width 0.2) (layer "B.Cu") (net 5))
 (segment (start 124.587 41.656) (end 125.095 41.148) (width 0.2) (layer "B.Cu") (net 5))
 (segment (start 102.616 55.245) (end 102.87 54.991) (width 0.2) (layer "B.Cu") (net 5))
 (segment (start 128.143 36.322) (end 136.144 36.322) (width 0.2) (layer "B.Cu") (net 5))
 (segment (start 136.779 35.687) (end 133.35 32.258) (width 0.2) (layer "B.Cu") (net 5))
 (segment (start 118.491 41.91) (end 118.618 41.783) (width 0.2) (layer "B.Cu") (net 5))
 (segment (start 102.616 62.23) (end 102.616 55.245) (width 0.2) (layer "B.Cu") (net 5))
 (segment (start 105.537 62.611) (end 102.997 62.611) (width 0.2) (layer "B.Cu") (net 5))
 (segment (start 118.491 54.991) (end 119.888 54.991) (width 0.2) (layer "B.Cu") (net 5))
 (segment (start 119.888 54.991) (end 120.523 55.626) (width 0.2) (layer "B.Cu") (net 5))
 (segment (start 125.095 36.576) (end 125.349 36.322) (width 0.2) (layer "B.Cu") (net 5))
 (segment (start 133.35 32.258) (end 133.35 23.368) (width 0.2) (layer "B.Cu") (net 5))
 (segment (start 119.176 27.827) (end 117.207 27.827) (width 0.2) (layer "F.Cu") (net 4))
 (segment (start 116.713 28.321) (end 116.713 32.125499) (width 0.2) (layer "F.Cu") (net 4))
 (segment (start 117.207 27.827) (end 116.713 28.321) (width 0.2) (layer "F.Cu") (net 4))
 (segment (start 119.176 27.827) (end 118.876 27.527) (width 0.2) (layer "F.Cu") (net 4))
 (segment (start 102.5281 21.991) (end 117.221 21.991) (width 0.2) (layer "F.Cu") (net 4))
 (segment (start 102.509 22.0589) (end 102.4846 22.0345) (width 0.2) (layer "F.Cu") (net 4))
 (segment (start 122.598999 53.6385) (end 122.598999 52.862555) (width 0.2) (layer "F.Cu") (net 4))
 (segment (start 102.4846 22.0345) (end 102.5281 21.991) (width 0.2) (layer "F.Cu") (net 4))
 (segment (start 102.509 22.586) (end 102.509 22.0589) (width 0.2) (layer "F.Cu") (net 4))
 (segment (start 102.3915 51.7865) (end 102.235 51.943) (width 0.2) (layer "F.Cu") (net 4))
 (segment (start 122.598999 52.862555) (end 121.522944 51.7865) (width 0.2) (layer "F.Cu") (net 4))
 (segment (start 118.876 27.527) (end 118.476 27.527) (width 0.2) (layer "F.Cu") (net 4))
 (segment (start 102.235 22.86) (end 102.509 22.586) (width 0.2) (layer "F.Cu") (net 4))
 (segment (start 117.221 27.813) (end 117.207 27.827) (width 0.2) (layer "F.Cu") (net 4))
 (segment (start 121.522944 51.7865) (end 102.3915 51.7865) (width 0.2) (layer "F.Cu") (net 4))
 (segment (start 121.474999 54.7625) (end 122.598999 53.6385) (width 0.2) (layer "F.Cu") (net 4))
 (segment (start 120.7375 54.7625) (end 121.474999 54.7625) (width 0.2) (layer "F.Cu") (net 4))
 (segment (start 117.221 21.991) (end 117.221 27.813) (width 0.2) (layer "F.Cu") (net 4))
 (segment (start 116.713 32.125499) (end 121.537501 36.95) (width 0.2) (layer "F.Cu") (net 4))
 (segment (start 121.537501 36.95) (end 122.275 36.95) (width 0.2) (layer "F.Cu") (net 4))
 (segment (start 102.235 51.943) (end 102.235 22.86) (width 0.2) (layer "F.Cu") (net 4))
 (segment (start 173.5 26.5) (end 192 26.5) (width 0.2) (layer "F.Cu") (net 19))
 (segment (start 172.96 25.96) (end 173.5 26.5) (width 0.2) (layer "F.Cu") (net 19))
 (segment (start 191.5 62) (end 131.215 62) (width 0.2) (layer "F.Cu") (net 19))
 (segment (start 172.96 24.5) (end 172.96 25.96) (width 0.2) (layer "F.Cu") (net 19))
 (segment (start 130.81 56.388) (end 130.7845 56.3625) (width 0.2) (layer "F.Cu") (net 19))
 (segment (start 192 61.5) (end 191.5 62) (width 0.2) (layer "F.Cu") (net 19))
 (segment (start 130.7845 56.3625) (end 129.0625 56.3625) (width 0.2) (layer "F.Cu") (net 19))
 (segment (start 131.064 61.849) (end 131.064 56.388) (width 0.2) (layer "F.Cu") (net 19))
 (segment (start 192 26.5) (end 192 61.5) (width 0.2) (layer "F.Cu") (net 19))
 (segment (start 131.064 56.388) (end 130.81 56.388) (width 0.2) (layer "F.Cu") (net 19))
 (segment (start 131.215 62) (end 131.064 61.849) (width 0.2) (layer "F.Cu") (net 19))
 (segment (start 193 24) (end 193 63) (width 0.2) (layer "F.Cu") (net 13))
 (segment (start 192.5 24.5) (end 193 24) (width 0.2) (layer "F.Cu") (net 13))
 (segment (start 125 63) (end 125.3 62.7) (width 0.2) (layer "F.Cu") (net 13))
 (segment (start 125.3 62.7) (end 125.3 59.325) (width 0.2) (layer "F.Cu") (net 13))
 (segment (start 193 63) (end 125 63) (width 0.2) (layer "F.Cu") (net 13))
 (segment (start 175.5 24.5) (end 192.5 24.5) (width 0.2) (layer "F.Cu") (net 13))
 (segment (start 171.958 53.975) (end 170.42 52.437) (width 0.2) (layer "F.Cu") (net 22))
 (segment (start 137.2365 53.1625) (end 137.414 53.34) (width 0.2) (layer "F.Cu") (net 22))
 (segment (start 189.992 53.975) (end 171.958 53.975) (width 0.2) (layer "F.Cu") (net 22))
 (segment (start 129.0625 53.1625) (end 137.2365 53.1625) (width 0.2) (layer "F.Cu") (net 22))
 (segment (start 137.414 60.96) (end 190.5 60.96) (width 0.2) (layer "F.Cu") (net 22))
 (segment (start 190.5 60.96) (end 190.754 60.706) (width 0.2) (layer "F.Cu") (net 22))
 (segment (start 170.42 52.437) (end 170.42 39.74) (width 0.2) (layer "F.Cu") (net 22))
 (segment (start 190.754 60.706) (end 190.754 54.737) (width 0.2) (layer "F.Cu") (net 22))
 (segment (start 137.414 53.34) (end 137.414 60.96) (width 0.2) (layer "F.Cu") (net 22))
 (segment (start 190.754 54.737) (end 189.992 53.975) (width 0.2) (layer "F.Cu") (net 22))
 (segment (start 127 62.5) (end 127 62) (width 0.2) (layer "F.Cu") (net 15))
 (segment (start 126.9 61.9) (end 126.9 59.325) (width 0.2) (layer "F.Cu") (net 15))
 (segment (start 191 62.5) (end 127 62.5) (width 0.2) (layer "F.Cu") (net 15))
 (segment (start 127 62) (end 126.9 61.9) (width 0.2) (layer "F.Cu") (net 15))
 (segment (start 119.176 25.527) (end 125.476 25.527) (width 0.2) (layer "F.Cu") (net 37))
 (segment (start 125.476 25.4679) (end 125.476 25.527) (width 0.2) (layer "F.Cu") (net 37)))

